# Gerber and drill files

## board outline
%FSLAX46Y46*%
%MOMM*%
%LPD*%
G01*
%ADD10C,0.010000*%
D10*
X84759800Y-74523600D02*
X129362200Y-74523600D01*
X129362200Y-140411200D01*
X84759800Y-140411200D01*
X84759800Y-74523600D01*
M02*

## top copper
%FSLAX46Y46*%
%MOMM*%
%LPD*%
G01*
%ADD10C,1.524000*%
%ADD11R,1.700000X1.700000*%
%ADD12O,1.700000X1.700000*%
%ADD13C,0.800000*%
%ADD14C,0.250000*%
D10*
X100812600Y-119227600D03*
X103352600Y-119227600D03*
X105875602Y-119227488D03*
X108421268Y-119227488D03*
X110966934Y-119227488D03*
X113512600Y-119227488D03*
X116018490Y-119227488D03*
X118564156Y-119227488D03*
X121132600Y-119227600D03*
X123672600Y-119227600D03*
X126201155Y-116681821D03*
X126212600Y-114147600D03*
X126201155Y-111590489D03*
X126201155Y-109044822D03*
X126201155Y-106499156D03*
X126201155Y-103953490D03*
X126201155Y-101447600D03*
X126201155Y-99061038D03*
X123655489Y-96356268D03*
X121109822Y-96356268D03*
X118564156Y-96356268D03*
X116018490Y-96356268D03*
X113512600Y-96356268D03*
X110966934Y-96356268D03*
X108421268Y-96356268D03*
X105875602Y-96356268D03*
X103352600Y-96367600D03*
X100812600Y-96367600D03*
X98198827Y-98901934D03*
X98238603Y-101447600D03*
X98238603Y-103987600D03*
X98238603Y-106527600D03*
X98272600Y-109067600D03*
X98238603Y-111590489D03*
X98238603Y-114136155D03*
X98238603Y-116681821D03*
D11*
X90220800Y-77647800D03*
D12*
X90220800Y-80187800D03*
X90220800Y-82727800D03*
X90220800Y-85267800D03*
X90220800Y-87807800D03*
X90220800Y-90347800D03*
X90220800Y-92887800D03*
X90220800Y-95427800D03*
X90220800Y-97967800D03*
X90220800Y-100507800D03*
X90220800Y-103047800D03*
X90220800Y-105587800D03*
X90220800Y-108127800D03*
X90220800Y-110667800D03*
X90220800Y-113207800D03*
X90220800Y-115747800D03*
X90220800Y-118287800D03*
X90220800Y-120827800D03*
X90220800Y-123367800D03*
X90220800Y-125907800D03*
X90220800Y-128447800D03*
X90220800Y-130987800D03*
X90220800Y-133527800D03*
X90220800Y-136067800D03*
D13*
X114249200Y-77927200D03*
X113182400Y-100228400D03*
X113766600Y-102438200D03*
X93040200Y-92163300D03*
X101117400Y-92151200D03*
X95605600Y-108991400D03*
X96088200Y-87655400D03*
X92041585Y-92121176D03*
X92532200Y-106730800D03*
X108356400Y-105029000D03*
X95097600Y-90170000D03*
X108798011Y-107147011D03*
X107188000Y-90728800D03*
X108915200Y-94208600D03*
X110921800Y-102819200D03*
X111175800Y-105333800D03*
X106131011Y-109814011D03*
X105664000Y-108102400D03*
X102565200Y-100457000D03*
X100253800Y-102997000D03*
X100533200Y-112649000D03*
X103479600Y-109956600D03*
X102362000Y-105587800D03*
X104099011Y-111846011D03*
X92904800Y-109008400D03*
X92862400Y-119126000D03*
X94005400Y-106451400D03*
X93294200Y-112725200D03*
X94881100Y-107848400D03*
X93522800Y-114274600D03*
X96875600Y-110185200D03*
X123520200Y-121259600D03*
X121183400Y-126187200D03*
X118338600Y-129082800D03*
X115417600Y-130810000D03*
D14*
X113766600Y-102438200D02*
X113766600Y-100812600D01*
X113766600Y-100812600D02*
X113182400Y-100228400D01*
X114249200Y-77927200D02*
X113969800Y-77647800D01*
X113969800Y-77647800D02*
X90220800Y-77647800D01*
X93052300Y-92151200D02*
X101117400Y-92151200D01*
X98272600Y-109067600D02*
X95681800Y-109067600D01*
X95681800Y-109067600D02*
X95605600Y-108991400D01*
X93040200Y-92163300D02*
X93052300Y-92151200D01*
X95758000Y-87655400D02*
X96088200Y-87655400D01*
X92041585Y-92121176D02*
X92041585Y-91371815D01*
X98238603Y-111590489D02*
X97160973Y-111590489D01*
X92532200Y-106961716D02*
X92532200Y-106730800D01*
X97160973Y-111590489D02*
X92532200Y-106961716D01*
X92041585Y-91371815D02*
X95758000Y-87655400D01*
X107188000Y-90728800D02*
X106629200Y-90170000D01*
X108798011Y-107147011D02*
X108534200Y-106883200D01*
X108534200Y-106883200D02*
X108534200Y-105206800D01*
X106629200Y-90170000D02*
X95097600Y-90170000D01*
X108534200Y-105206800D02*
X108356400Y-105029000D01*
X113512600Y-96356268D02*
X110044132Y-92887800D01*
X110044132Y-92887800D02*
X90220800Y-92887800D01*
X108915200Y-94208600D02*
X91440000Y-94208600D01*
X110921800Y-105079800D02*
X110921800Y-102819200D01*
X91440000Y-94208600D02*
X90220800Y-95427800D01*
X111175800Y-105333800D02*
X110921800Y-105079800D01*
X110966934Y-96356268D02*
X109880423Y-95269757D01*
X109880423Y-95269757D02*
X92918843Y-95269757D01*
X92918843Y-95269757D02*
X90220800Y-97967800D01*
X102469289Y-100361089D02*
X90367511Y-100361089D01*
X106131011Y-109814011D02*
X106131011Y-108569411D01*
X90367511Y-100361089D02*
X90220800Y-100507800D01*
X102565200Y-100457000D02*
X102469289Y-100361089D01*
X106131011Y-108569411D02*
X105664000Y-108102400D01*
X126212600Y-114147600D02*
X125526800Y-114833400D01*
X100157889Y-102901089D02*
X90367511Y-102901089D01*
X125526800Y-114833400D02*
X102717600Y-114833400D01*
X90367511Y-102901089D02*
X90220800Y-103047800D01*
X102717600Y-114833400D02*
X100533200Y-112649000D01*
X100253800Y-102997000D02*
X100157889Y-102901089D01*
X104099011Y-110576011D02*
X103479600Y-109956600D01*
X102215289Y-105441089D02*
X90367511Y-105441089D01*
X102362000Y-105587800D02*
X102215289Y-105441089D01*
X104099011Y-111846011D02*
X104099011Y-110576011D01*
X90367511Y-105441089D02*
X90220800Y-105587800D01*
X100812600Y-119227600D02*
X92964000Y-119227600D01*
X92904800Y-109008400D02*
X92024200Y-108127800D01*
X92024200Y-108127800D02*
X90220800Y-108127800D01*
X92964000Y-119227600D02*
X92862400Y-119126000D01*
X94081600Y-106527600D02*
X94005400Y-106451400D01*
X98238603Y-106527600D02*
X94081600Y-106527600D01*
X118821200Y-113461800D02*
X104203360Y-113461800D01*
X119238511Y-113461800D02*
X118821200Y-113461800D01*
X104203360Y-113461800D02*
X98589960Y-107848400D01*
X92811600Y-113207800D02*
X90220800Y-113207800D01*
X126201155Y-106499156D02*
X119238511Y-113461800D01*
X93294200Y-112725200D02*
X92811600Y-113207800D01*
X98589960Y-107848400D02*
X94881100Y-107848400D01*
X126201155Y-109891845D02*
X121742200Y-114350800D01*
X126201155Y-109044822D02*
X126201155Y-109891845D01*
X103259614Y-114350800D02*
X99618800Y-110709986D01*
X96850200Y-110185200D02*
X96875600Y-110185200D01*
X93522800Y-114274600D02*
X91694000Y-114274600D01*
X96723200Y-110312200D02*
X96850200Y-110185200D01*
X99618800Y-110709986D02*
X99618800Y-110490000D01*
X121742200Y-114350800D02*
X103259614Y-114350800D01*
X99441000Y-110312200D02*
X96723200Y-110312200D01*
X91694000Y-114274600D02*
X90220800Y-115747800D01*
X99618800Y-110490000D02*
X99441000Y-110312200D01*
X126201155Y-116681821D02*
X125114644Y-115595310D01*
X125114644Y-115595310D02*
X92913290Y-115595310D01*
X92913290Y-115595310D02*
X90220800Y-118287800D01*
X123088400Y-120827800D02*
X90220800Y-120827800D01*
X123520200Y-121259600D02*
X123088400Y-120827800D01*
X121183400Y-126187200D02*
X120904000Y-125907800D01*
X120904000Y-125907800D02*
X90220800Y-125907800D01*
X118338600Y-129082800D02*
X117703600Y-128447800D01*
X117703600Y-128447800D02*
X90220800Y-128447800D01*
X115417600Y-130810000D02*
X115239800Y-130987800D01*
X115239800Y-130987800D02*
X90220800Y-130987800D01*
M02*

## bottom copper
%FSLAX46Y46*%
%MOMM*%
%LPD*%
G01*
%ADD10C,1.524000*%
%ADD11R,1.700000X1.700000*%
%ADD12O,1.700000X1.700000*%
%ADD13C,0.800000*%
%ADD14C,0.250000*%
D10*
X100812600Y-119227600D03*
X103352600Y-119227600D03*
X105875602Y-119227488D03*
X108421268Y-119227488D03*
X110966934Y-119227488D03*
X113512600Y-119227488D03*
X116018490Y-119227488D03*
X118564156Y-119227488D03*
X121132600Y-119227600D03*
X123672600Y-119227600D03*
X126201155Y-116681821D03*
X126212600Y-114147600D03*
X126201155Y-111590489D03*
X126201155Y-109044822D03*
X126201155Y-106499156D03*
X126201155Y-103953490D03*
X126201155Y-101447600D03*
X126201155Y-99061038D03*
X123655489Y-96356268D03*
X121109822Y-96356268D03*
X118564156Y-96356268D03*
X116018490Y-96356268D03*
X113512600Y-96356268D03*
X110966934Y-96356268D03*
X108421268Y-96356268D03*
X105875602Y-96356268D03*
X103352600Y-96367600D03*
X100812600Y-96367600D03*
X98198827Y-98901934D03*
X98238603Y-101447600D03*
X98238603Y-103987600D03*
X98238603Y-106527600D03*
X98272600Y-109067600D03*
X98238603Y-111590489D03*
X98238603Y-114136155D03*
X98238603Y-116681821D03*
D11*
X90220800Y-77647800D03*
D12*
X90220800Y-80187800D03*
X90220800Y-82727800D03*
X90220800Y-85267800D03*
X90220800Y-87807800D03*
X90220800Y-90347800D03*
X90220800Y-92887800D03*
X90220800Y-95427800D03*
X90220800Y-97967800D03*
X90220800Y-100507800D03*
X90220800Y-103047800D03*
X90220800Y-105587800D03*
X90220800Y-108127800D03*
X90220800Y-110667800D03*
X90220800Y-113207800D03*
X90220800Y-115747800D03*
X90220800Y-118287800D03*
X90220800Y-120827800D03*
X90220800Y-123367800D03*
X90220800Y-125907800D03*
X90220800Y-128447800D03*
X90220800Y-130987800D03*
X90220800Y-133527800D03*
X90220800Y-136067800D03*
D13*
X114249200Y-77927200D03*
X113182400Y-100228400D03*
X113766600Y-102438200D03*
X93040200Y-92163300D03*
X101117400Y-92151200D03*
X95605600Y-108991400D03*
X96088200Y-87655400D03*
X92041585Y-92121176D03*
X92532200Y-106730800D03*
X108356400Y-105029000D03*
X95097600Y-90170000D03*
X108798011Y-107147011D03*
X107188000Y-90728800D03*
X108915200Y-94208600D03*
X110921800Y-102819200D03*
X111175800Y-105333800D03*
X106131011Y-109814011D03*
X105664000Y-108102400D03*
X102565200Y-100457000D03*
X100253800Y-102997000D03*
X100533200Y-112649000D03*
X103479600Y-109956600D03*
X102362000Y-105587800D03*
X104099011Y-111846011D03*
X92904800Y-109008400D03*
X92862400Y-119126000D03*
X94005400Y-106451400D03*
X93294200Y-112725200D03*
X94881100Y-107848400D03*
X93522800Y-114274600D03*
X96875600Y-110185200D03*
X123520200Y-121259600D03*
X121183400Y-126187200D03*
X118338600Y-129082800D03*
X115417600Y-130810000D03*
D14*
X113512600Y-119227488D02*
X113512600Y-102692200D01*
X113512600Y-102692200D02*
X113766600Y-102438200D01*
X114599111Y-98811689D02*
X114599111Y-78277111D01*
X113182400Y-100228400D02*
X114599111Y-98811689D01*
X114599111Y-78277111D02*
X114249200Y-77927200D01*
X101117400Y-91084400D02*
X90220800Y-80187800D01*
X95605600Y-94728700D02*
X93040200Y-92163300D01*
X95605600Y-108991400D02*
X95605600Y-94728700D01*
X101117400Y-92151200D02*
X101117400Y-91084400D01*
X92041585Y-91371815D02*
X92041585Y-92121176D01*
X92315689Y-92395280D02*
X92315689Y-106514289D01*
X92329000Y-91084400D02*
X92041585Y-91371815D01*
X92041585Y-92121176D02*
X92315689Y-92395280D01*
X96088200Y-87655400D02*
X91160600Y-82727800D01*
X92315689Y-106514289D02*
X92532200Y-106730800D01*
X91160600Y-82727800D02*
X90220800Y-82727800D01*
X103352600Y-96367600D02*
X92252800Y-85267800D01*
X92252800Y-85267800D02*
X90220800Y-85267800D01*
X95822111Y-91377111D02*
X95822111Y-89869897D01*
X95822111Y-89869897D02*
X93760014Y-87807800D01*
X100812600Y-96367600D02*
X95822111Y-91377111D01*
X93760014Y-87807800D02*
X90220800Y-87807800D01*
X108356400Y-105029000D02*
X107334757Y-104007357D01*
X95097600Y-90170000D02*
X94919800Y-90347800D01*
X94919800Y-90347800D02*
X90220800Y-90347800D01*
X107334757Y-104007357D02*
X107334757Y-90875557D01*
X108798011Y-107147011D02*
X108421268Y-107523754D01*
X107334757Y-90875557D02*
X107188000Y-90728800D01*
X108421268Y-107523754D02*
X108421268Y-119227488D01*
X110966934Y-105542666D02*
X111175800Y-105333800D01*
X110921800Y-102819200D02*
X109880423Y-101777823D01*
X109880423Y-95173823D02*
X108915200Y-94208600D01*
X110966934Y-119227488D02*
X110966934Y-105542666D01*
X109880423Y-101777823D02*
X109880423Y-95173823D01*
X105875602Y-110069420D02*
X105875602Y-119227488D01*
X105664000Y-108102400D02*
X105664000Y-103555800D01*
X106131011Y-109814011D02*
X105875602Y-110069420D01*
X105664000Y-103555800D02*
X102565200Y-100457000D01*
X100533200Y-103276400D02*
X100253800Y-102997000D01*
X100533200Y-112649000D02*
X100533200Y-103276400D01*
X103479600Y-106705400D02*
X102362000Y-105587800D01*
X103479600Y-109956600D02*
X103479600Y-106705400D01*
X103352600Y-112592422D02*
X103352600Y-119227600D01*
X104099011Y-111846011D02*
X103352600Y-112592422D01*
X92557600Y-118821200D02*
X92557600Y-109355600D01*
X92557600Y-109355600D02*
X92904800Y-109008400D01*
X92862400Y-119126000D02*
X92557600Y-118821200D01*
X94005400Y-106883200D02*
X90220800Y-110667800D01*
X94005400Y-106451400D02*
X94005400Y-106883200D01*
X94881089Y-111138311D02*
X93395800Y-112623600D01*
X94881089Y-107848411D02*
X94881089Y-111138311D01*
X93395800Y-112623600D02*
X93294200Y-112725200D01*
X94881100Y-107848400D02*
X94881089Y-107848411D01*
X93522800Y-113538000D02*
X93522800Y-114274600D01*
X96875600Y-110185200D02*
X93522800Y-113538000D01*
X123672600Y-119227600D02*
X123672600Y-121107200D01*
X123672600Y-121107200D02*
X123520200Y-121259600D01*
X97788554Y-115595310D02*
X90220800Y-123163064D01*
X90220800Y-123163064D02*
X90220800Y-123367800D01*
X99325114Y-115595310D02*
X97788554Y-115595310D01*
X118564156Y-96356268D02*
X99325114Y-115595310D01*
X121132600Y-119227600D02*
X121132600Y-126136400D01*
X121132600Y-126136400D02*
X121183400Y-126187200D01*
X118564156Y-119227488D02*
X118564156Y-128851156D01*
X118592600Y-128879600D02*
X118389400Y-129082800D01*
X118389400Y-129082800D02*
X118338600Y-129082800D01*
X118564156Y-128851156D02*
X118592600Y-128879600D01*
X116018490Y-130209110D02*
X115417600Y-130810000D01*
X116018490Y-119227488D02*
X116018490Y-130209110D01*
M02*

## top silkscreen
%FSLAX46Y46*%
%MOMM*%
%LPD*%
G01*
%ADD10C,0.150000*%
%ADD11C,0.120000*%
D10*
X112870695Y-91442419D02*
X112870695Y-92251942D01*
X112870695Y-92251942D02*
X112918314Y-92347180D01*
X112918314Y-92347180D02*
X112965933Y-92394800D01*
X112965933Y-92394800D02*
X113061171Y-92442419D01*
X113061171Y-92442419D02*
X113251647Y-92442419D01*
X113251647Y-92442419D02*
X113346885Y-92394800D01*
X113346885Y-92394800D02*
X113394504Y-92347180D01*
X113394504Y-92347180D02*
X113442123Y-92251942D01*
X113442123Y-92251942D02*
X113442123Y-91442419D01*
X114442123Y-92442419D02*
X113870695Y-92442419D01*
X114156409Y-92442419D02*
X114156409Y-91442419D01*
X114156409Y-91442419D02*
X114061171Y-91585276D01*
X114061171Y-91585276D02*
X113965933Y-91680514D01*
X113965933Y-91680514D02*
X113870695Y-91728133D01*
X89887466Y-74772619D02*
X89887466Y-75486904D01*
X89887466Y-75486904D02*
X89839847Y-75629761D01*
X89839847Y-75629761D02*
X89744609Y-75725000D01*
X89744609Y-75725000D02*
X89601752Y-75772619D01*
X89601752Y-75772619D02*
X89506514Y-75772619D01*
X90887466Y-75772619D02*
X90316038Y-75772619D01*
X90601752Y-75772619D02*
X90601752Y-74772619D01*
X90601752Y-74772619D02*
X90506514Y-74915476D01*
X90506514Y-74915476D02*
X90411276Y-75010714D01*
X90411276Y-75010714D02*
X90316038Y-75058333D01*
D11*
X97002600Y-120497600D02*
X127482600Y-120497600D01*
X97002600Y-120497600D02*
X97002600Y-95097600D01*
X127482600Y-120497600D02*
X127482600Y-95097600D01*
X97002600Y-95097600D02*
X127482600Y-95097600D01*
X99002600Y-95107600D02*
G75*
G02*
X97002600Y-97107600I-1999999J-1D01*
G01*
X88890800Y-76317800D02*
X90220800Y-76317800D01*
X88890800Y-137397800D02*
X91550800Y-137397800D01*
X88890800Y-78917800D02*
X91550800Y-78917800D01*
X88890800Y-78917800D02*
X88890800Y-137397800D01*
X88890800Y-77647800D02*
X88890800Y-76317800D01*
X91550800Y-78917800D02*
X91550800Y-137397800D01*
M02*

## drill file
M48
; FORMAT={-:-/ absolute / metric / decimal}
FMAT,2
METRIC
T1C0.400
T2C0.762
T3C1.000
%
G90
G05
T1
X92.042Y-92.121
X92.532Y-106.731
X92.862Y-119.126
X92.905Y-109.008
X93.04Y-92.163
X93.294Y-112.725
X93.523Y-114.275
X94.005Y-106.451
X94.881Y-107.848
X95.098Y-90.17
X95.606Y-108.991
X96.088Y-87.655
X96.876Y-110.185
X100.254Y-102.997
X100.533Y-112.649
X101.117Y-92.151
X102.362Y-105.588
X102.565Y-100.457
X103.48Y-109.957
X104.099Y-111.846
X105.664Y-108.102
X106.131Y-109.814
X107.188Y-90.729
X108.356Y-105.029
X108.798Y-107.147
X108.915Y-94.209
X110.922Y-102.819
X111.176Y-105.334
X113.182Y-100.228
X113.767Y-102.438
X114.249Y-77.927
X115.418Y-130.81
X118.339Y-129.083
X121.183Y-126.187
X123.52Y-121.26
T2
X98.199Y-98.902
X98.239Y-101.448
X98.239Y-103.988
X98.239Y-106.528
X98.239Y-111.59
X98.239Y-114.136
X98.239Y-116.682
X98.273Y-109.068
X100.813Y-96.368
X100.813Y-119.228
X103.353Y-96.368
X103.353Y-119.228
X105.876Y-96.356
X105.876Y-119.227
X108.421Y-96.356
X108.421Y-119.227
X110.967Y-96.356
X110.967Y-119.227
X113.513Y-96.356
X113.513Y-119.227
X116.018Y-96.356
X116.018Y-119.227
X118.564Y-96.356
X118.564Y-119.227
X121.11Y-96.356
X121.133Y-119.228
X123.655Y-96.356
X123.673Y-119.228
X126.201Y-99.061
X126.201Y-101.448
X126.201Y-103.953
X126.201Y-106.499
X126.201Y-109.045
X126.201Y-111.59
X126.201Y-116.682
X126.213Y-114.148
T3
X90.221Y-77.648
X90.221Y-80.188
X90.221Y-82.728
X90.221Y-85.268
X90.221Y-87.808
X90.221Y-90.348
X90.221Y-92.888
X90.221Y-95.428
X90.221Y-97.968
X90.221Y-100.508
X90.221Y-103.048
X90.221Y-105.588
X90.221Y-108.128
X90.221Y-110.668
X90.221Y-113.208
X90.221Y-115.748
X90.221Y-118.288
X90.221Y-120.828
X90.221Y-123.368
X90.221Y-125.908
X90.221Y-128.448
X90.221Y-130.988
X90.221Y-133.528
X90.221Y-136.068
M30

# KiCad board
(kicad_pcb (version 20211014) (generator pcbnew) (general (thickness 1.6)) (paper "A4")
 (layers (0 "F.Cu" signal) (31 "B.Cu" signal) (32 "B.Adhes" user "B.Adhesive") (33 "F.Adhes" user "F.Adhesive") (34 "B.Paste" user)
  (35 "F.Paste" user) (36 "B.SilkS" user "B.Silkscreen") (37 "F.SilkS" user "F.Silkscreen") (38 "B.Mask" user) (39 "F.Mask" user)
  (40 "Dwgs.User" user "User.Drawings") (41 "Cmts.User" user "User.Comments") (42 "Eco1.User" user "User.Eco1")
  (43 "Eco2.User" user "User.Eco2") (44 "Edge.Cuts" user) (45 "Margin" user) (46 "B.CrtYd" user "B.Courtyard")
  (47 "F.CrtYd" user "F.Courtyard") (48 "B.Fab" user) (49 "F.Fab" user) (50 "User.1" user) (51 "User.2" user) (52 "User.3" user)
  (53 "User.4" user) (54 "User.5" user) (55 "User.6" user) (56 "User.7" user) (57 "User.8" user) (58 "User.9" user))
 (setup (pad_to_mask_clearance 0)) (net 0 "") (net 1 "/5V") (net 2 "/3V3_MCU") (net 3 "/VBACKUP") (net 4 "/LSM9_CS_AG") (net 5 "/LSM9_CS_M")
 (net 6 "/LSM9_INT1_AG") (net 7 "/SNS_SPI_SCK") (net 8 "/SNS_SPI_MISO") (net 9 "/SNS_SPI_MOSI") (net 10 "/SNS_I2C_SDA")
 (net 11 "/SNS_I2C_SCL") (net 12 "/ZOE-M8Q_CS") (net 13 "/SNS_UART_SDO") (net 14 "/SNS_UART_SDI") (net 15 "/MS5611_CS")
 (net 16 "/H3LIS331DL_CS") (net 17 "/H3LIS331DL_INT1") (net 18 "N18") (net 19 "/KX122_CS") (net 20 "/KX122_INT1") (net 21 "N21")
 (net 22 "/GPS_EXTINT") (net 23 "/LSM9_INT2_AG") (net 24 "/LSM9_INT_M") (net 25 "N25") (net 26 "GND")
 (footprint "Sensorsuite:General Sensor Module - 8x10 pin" (layer "F.Cu") (at 113.5126 106.5276)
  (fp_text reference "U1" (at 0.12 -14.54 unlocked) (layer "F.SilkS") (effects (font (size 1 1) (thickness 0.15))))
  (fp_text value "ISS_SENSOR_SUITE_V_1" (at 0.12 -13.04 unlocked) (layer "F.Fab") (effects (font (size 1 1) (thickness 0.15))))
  (fp_line (start -16.51 13.97) (end 13.97 13.97) (layer "F.SilkS") (width 0.12))
  (fp_line (start -16.51 13.97) (end -16.51 -11.43) (layer "F.SilkS") (width 0.12))
  (fp_line (start 13.97 13.97) (end 13.97 -11.43) (layer "F.SilkS") (width 0.12))
  (fp_line (start -16.51 -11.43) (end 13.97 -11.43) (layer "F.SilkS") (width 0.12))
  (fp_arc (start -14.51 -11.42) (mid -15.095786 -10.005786) (end -16.51 -9.42) (layer "F.SilkS") (width 0.12))
  (pad "1" thru_hole circle (at -12.7 12.7) (size 1.524 1.524) (drill 0.762) (layers *.Cu *.Mask) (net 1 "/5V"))
  (pad "2" thru_hole circle (at -10.16 12.7) (size 1.524 1.524) (drill 0.762) (layers *.Cu *.Mask) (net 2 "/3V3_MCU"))
  (pad "3" thru_hole circle (at -7.636998 12.699888) (size 1.524 1.524) (drill 0.762) (layers *.Cu *.Mask) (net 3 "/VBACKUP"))
  (pad "4" thru_hole circle (at -5.091332 12.699888) (size 1.524 1.524) (drill 0.762) (layers *.Cu *.Mask) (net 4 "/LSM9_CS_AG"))
  (pad "5" thru_hole circle (at -2.545666 12.699888) (size 1.524 1.524) (drill 0.762) (layers *.Cu *.Mask) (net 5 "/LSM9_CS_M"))
  (pad "6" thru_hole circle (at 0 12.699888) (size 1.524 1.524) (drill 0.762) (layers *.Cu *.Mask) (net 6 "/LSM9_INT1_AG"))
  (pad "7" thru_hole circle (at 2.50589 12.699888) (size 1.524 1.524) (drill 0.762) (layers *.Cu *.Mask) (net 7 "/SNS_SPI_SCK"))
  (pad "8" thru_hole circle (at 5.051556 12.699888) (size 1.524 1.524) (drill 0.762) (layers *.Cu *.Mask) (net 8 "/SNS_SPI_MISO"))
  (pad "9" thru_hole circle (at 7.62 12.7) (size 1.524 1.524) (drill 0.762) (layers *.Cu *.Mask) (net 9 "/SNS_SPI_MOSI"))
  (pad "10" thru_hole circle (at 10.16 12.7) (size 1.524 1.524) (drill 0.762) (layers *.Cu *.Mask) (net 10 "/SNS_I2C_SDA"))
  (pad "11" thru_hole circle (at 12.688555 10.154221) (size 1.524 1.524) (drill 0.762) (layers *.Cu *.Mask) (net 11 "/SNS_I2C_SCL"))
  (pad "12" thru_hole circle (at 12.7 7.62) (size 1.524 1.524) (drill 0.762) (layers *.Cu *.Mask) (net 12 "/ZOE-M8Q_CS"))
  (pad "13" thru_hole circle (at 12.688555 5.062889) (size 1.524 1.524) (drill 0.762) (layers *.Cu *.Mask))
  (pad "14" thru_hole circle (at 12.688555 2.517222) (size 1.524 1.524) (drill 0.762) (layers *.Cu *.Mask) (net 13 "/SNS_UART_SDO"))
  (pad "15" thru_hole circle (at 12.688555 -0.028444) (size 1.524 1.524) (drill 0.762) (layers *.Cu *.Mask) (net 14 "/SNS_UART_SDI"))
  (pad "16" thru_hole circle (at 12.688555 -2.57411) (size 1.524 1.524) (drill 0.762) (layers *.Cu *.Mask))
  (pad "17" thru_hole circle (at 12.688555 -5.08) (size 1.524 1.524) (drill 0.762) (layers *.Cu *.Mask))
  (pad "18" thru_hole circle (at 12.688555 -7.466562) (size 1.524 1.524) (drill 0.762) (layers *.Cu *.Mask))
  (pad "19" thru_hole circle (at 10.142889 -10.171332) (size 1.524 1.524) (drill 0.762) (layers *.Cu *.Mask))
  (pad "20" thru_hole circle (at 7.597222 -10.171332) (size 1.524 1.524) (drill 0.762) (layers *.Cu *.Mask))
  (pad "21" thru_hole circle (at 5.051556 -10.171332) (size 1.524 1.524) (drill 0.762) (layers *.Cu *.Mask) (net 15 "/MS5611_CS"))
  (pad "22" thru_hole circle (at 2.50589 -10.171332) (size 1.524 1.524) (drill 0.762) (layers *.Cu *.Mask))
  (pad "23" thru_hole circle (at 0 -10.171332) (size 1.524 1.524) (drill 0.762) (layers *.Cu *.Mask) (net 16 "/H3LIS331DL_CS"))
  (pad "24" thru_hole circle (at -2.545666 -10.171332) (size 1.524 1.524) (drill 0.762) (layers *.Cu *.Mask) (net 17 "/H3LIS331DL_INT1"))
  (pad "25" thru_hole circle (at -5.091332 -10.171332) (size 1.524 1.524) (drill 0.762) (layers *.Cu *.Mask))
  (pad "26" thru_hole circle (at -7.636998 -10.171332) (size 1.524 1.524) (drill 0.762) (layers *.Cu *.Mask) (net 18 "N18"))
  (pad "27" thru_hole circle (at -10.16 -10.16) (size 1.524 1.524) (drill 0.762) (layers *.Cu *.Mask) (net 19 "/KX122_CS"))
  (pad "28" thru_hole circle (at -12.7 -10.16) (size 1.524 1.524) (drill 0.762) (layers *.Cu *.Mask) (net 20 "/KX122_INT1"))
  (pad "29" thru_hole circle (at -15.313773 -7.625666) (size 1.524 1.524) (drill 0.762) (layers *.Cu *.Mask))
  (pad "30" thru_hole circle (at -15.273997 -5.08) (size 1.524 1.524) (drill 0.762) (layers *.Cu *.Mask))
  (pad "31" thru_hole circle (at -15.273997 -2.54) (size 1.524 1.524) (drill 0.762) (layers *.Cu *.Mask) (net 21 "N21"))
  (pad "32" thru_hole circle (at -15.273997 0) (size 1.524 1.524) (drill 0.762) (layers *.Cu *.Mask) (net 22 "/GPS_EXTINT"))
  (pad "33" thru_hole circle (at -15.24 2.54) (size 1.524 1.524) (drill 0.762) (layers *.Cu *.Mask) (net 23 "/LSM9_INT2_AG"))
  (pad "34" thru_hole circle (at -15.273997 5.062889) (size 1.524 1.524) (drill 0.762) (layers *.Cu *.Mask) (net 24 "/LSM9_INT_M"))
  (pad "35" thru_hole circle (at -15.273997 7.608555) (size 1.524 1.524) (drill 0.762) (layers *.Cu *.Mask))
  (pad "36" thru_hole circle (at -15.273997 10.154221) (size 1.524 1.524) (drill 0.762) (layers *.Cu *.Mask)))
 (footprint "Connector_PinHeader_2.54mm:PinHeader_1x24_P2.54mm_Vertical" (layer "F.Cu") (at 90.2208 77.6478)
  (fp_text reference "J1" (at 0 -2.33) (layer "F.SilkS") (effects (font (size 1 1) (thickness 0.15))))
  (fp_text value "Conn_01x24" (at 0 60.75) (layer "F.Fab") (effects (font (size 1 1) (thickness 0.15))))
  (fp_line (start -1.33 -1.33) (end 0 -1.33) (layer "F.SilkS") (width 0.12))
  (fp_line (start -1.33 59.75) (end 1.33 59.75) (layer "F.SilkS") (width 0.12))
  (fp_line (start -1.33 1.27) (end 1.33 1.27) (layer "F.SilkS") (width 0.12))
  (fp_line (start -1.33 1.27) (end -1.33 59.75) (layer "F.SilkS") (width 0.12))
  (fp_line (start -1.33 0) (end -1.33 -1.33) (layer "F.SilkS") (width 0.12))
  (fp_line (start 1.33 1.27) (end 1.33 59.75) (layer "F.SilkS") (width 0.12))
  (pad "1" thru_hole rect locked (at 0 0) (size 1.7 1.7) (drill 1) (layers *.Cu *.Mask) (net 6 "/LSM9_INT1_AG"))
  (pad "2" thru_hole oval locked (at 0 2.54) (size 1.7 1.7) (drill 1) (layers *.Cu *.Mask) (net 23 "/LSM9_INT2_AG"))
  (pad "3" thru_hole oval locked (at 0 5.08) (size 1.7 1.7) (drill 1) (layers *.Cu *.Mask) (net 24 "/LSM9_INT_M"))
  (pad "4" thru_hole oval locked (at 0 7.62) (size 1.7 1.7) (drill 1) (layers *.Cu *.Mask) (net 19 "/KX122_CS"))
  (pad "5" thru_hole oval locked (at 0 10.16) (size 1.7 1.7) (drill 1) (layers *.Cu *.Mask) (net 20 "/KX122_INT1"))
  (pad "6" thru_hole oval locked (at 0 12.7) (size 1.7 1.7) (drill 1) (layers *.Cu *.Mask) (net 4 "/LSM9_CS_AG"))
  (pad "7" thru_hole oval locked (at 0 15.24) (size 1.7 1.7) (drill 1) (layers *.Cu *.Mask) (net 16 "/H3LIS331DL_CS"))
  (pad "8" thru_hole oval locked (at 0 17.78) (size 1.7 1.7) (drill 1) (layers *.Cu *.Mask) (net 5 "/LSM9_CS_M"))
  (pad "9" thru_hole oval locked (at 0 20.32) (size 1.7 1.7) (drill 1) (layers *.Cu *.Mask) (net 17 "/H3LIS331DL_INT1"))
  (pad "10" thru_hole oval locked (at 0 22.86) (size 1.7 1.7) (drill 1) (layers *.Cu *.Mask) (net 3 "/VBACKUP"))
  (pad "11" thru_hole oval locked (at 0 25.4) (size 1.7 1.7) (drill 1) (layers *.Cu *.Mask) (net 12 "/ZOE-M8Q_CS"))
  (pad "12" thru_hole oval locked (at 0 27.94) (size 1.7 1.7) (drill 1) (layers *.Cu *.Mask) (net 2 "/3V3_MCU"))
  (pad "13" thru_hole oval locked (at 0 30.48) (size 1.7 1.7) (drill 1) (layers *.Cu *.Mask) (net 1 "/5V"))
  (pad "14" thru_hole oval locked (at 0 33.02) (size 1.7 1.7) (drill 1) (layers *.Cu *.Mask) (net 22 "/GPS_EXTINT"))
  (pad "15" thru_hole oval locked (at 0 35.56) (size 1.7 1.7) (drill 1) (layers *.Cu *.Mask) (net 14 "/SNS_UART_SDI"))
  (pad "16" thru_hole oval locked (at 0 38.1) (size 1.7 1.7) (drill 1) (layers *.Cu *.Mask) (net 13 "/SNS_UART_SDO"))
  (pad "17" thru_hole oval locked (at 0 40.64) (size 1.7 1.7) (drill 1) (layers *.Cu *.Mask) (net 11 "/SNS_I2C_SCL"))
  (pad "18" thru_hole oval locked (at 0 43.18) (size 1.7 1.7) (drill 1) (layers *.Cu *.Mask) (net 10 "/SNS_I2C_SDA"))
  (pad "19" thru_hole oval locked (at 0 45.72) (size 1.7 1.7) (drill 1) (layers *.Cu *.Mask) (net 15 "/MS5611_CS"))
  (pad "20" thru_hole oval locked (at 0 48.26) (size 1.7 1.7) (drill 1) (layers *.Cu *.Mask) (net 9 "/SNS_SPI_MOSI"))
  (pad "21" thru_hole oval locked (at 0 50.8) (size 1.7 1.7) (drill 1) (layers *.Cu *.Mask) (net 8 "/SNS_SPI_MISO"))
  (pad "22" thru_hole oval locked (at 0 53.34) (size 1.7 1.7) (drill 1) (layers *.Cu *.Mask) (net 7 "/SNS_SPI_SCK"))
  (pad "23" thru_hole oval locked (at 0 55.88) (size 1.7 1.7) (drill 1) (layers *.Cu *.Mask) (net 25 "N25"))
  (pad "24" thru_hole oval locked (at 0 58.42) (size 1.7 1.7) (drill 1) (layers *.Cu *.Mask) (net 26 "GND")))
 (gr_rect (start 84.7598 74.5236) (end 129.3622 140.4112) (layer "Edge.Cuts") (width 0.01) (fill none))
 (segment (start 113.7666 102.4382) (end 113.7666 100.8126) (width 0.25) (layer "F.Cu") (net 6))
 (segment (start 113.7666 100.8126) (end 113.1824 100.2284) (width 0.25) (layer "F.Cu") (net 6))
 (segment (start 114.2492 77.9272) (end 113.9698 77.6478) (width 0.25) (layer "F.Cu") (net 6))
 (segment (start 113.9698 77.6478) (end 90.2208 77.6478) (width 0.25) (layer "F.Cu") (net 6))
 (via (at 114.2492 77.9272) (size 0.8) (drill 0.4) (layers "F.Cu" "B.Cu") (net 6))
 (via (at 113.1824 100.2284) (size 0.8) (drill 0.4) (layers "F.Cu" "B.Cu") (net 6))
 (via (at 113.7666 102.4382) (size 0.8) (drill 0.4) (layers "F.Cu" "B.Cu") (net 6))
 (segment (start 113.5126 119.227488) (end 113.5126 102.6922) (width 0.25) (layer "B.Cu") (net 6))
 (segment (start 113.5126 102.6922) (end 113.7666 102.4382) (width 0.25) (layer "B.Cu") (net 6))
 (segment (start 114.599111 98.811689) (end 114.599111 78.277111) (width 0.25) (layer "B.Cu") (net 6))
 (segment (start 113.1824 100.2284) (end 114.599111 98.811689) (width 0.25) (layer "B.Cu") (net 6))
 (segment (start 114.599111 78.277111) (end 114.2492 77.9272) (width 0.25) (layer "B.Cu") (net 6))
 (segment (start 93.0523 92.1512) (end 101.1174 92.1512) (width 0.25) (layer "F.Cu") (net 23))
 (segment (start 98.2726 109.0676) (end 95.6818 109.0676) (width 0.25) (layer "F.Cu") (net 23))
 (segment (start 95.6818 109.0676) (end 95.6056 108.9914) (width 0.25) (layer "F.Cu") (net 23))
 (segment (start 93.0402 92.1633) (end 93.0523 92.1512) (width 0.25) (layer "F.Cu") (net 23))
 (via (at 93.0402 92.1633) (size 0.8) (drill 0.4) (layers "F.Cu" "B.Cu") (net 23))
 (via (at 101.1174 92.1512) (size 0.8) (drill 0.4) (layers "F.Cu" "B.Cu") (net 23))
 (via (at 95.6056 108.9914) (size 0.8) (drill 0.4) (layers "F.Cu" "B.Cu") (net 23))
 (segment (start 101.1174 91.0844) (end 90.2208 80.1878) (width 0.25) (layer "B.Cu") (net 23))
 (segment (start 95.6056 94.7287) (end 93.0402 92.1633) (width 0.25) (layer "B.Cu") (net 23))
 (segment (start 95.6056 108.9914) (end 95.6056 94.7287) (width 0.25) (layer "B.Cu") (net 23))
 (segment (start 101.1174 92.1512) (end 101.1174 91.0844) (width 0.25) (layer "B.Cu") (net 23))
 (segment (start 95.758 87.6554) (end 96.0882 87.6554) (width 0.25) (layer "F.Cu") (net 24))
 (segment (start 92.041585 92.121176) (end 92.041585 91.371815) (width 0.25) (layer "F.Cu") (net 24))
 (segment (start 98.238603 111.590489) (end 97.160973 111.590489) (width 0.25) (layer "F.Cu") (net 24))
 (segment (start 92.5322 106.961716) (end 92.5322 106.7308) (width 0.25) (layer "F.Cu") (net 24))
 (segment (start 97.160973 111.590489) (end 92.5322 106.961716) (width 0.25) (layer "F.Cu") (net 24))
 (segment (start 92.041585 91.371815) (end 95.758 87.6554) (width 0.25) (layer "F.Cu") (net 24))
 (via (at 96.0882 87.6554) (size 0.8) (drill 0.4) (layers "F.Cu" "B.Cu") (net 24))
 (via (at 92.041585 92.121176) (size 0.8) (drill 0.4) (layers "F.Cu" "B.Cu") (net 24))
 (via (at 92.5322 106.7308) (size 0.8) (drill 0.4) (layers "F.Cu" "B.Cu") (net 24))
 (segment (start 92.041585 91.371815) (end 92.041585 92.121176) (width 0.25) (layer "B.Cu") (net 24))
 (segment (start 92.315689 92.39528) (end 92.315689 106.514289) (width 0.25) (layer "B.Cu") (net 24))
 (segment (start 92.329 91.0844) (end 92.041585 91.371815) (width 0.25) (layer "B.Cu") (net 24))
 (segment (start 92.041585 92.121176) (end 92.315689 92.39528) (width 0.25) (layer "B.Cu") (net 24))
 (segment (start 96.0882 87.6554) (end 91.1606 82.7278) (width 0.25) (layer "B.Cu") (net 24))
 (segment (start 92.315689 106.514289) (end 92.5322 106.7308) (width 0.25) (layer "B.Cu") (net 24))
 (segment (start 91.1606 82.7278) (end 90.2208 82.7278) (width 0.25) (layer "B.Cu") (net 24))
 (segment (start 103.3526 96.3676) (end 92.2528 85.2678) (width 0.25) (layer "B.Cu") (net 19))
 (segment (start 92.2528 85.2678) (end 90.2208 85.2678) (width 0.25) (layer "B.Cu") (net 19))
 (segment (start 95.822111 91.377111) (end 95.822111 89.869897) (width 0.25) (layer "B.Cu") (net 20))
 (segment (start 95.822111 89.869897) (end 93.760014 87.8078) (width 0.25) (layer "B.Cu") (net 20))
 (segment (start 100.8126 96.3676) (end 95.822111 91.377111) (width 0.25) (layer "B.Cu") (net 20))
 (segment (start 93.760014 87.8078) (end 90.2208 87.8078) (width 0.25) (layer "B.Cu") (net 20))
 (segment (start 107.188 90.7288) (end 106.6292 90.17) (width 0.25) (layer "F.Cu") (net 4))
 (segment (start 108.798011 107.147011) (end 108.5342 106.8832) (width 0.25) (layer "F.Cu") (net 4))
 (segment (start 108.5342 106.8832) (end 108.5342 105.2068) (width 0.25) (layer "F.Cu") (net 4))
 (segment (start 106.6292 90.17) (end 95.0976 90.17) (width 0.25) (layer "F.Cu") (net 4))
 (segment (start 108.5342 105.2068) (end 108.3564 105.029) (width 0.25) (layer "F.Cu") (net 4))
 (via (at 108.3564 105.029) (size 0.8) (drill 0.4) (layers "F.Cu" "B.Cu") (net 4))
 (via (at 95.0976 90.17) (size 0.8) (drill 0.4) (layers "F.Cu" "B.Cu") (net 4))
 (via (at 108.798011 107.147011) (size 0.8) (drill 0.4) (layers "F.Cu" "B.Cu") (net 4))
 (via (at 107.188 90.7288) (size 0.8) (drill 0.4) (layers "F.Cu" "B.Cu") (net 4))
 (segment (start 108.3564 105.029) (end 107.334757 104.007357) (width 0.25) (layer "B.Cu") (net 4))
 (segment (start 95.0976 90.17) (end 94.9198 90.3478) (width 0.25) (layer "B.Cu") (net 4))
 (segment (start 94.9198 90.3478) (end 90.2208 90.3478) (width 0.25) (layer "B.Cu") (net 4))
 (segment (start 107.334757 104.007357) (end 107.334757 90.875557) (width 0.25) (layer "B.Cu") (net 4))
 (segment (start 108.798011 107.147011) (end 108.421268 107.523754) (width 0.25) (layer "B.Cu") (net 4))
 (segment (start 107.334757 90.875557) (end 107.188 90.7288) (width 0.25) (layer "B.Cu") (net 4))
 (segment (start 108.421268 107.523754) (end 108.421268 119.227488) (width 0.25) (layer "B.Cu") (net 4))
 (segment (start 113.5126 96.356268) (end 110.044132 92.8878) (width 0.25) (layer "F.Cu") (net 16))
 (segment (start 110.044132 92.8878) (end 90.2208 92.8878) (width 0.25) (layer "F.Cu") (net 16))
 (segment (start 108.9152 94.2086) (end 91.44 94.2086) (width 0.25) (layer "F.Cu") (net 5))
 (segment (start 110.9218 105.0798) (end 110.9218 102.8192) (width 0.25) (layer "F.Cu") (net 5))
 (segment (start 91.44 94.2086) (end 90.2208 95.4278) (width 0.25) (layer "F.Cu") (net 5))
 (segment (start 111.1758 105.3338) (end 110.9218 105.0798) (width 0.25) (layer "F.Cu") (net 5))
 (via (at 108.9152 94.2086) (size 0.8) (drill 0.4) (layers "F.Cu" "B.Cu") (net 5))
 (via (at 110.9218 102.8192) (size 0.8) (drill 0.4) (layers "F.Cu" "B.Cu") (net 5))
 (via (at 111.1758 105.3338) (size 0.8) (drill 0.4) (layers "F.Cu" "B.Cu") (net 5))
 (segment (start 110.966934 105.542666) (end 111.1758 105.3338) (width 0.25) (layer "B.Cu") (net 5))
 (segment (start 110.9218 102.8192) (end 109.880423 101.777823) (width 0.25) (layer "B.Cu") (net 5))
 (segment (start 109.880423 95.173823) (end 108.9152 94.2086) (width 0.25) (layer "B.Cu") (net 5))
 (segment (start 110.966934 119.227488) (end 110.966934 105.542666) (width 0.25) (layer "B.Cu") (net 5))
 (segment (start 109.880423 101.777823) (end 109.880423 95.173823) (width 0.25) (layer "B.Cu") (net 5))
 (segment (start 110.966934 96.356268) (end 109.880423 95.269757) (width 0.25) (layer "F.Cu") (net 17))
 (segment (start 109.880423 95.269757) (end 92.918843 95.269757) (width 0.25) (layer "F.Cu") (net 17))
 (segment (start 92.918843 95.269757) (end 90.2208 97.9678) (width 0.25) (layer "F.Cu") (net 17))
 (segment (start 102.469289 100.361089) (end 90.367511 100.361089) (width 0.25) (layer "F.Cu") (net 3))
 (segment (start 106.131011 109.814011) (end 106.131011 108.569411) (width 0.25) (layer "F.Cu") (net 3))
 (segment (start 90.367511 100.361089) (end 90.2208 100.5078) (width 0.25) (layer "F.Cu") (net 3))
 (segment (start 102.5652 100.457) (end 102.469289 100.361089) (width 0.25) (layer "F.Cu") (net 3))
 (segment (start 106.131011 108.569411) (end 105.664 108.1024) (width 0.25) (layer "F.Cu") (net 3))
 (via (at 106.131011 109.814011) (size 0.8) (drill 0.4) (layers "F.Cu" "B.Cu") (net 3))
 (via (at 105.664 108.1024) (size 0.8) (drill 0.4) (layers "F.Cu" "B.Cu") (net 3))
 (via (at 102.5652 100.457) (size 0.8) (drill 0.4) (layers "F.Cu" "B.Cu") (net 3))
 (segment (start 105.875602 110.06942) (end 105.875602 119.227488) (width 0.25) (layer "B.Cu") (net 3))
 (segment (start 105.664 108.1024) (end 105.664 103.5558) (width 0.25) (layer "B.Cu") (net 3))
 (segment (start 106.131011 109.814011) (end 105.875602 110.06942) (width 0.25) (layer "B.Cu") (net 3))
 (segment (start 105.664 103.5558) (end 102.5652 100.457) (width 0.25) (layer "B.Cu") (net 3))
 (segment (start 126.2126 114.1476) (end 125.5268 114.8334) (width 0.25) (layer "F.Cu") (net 12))
 (segment (start 100.157889 102.901089) (end 90.367511 102.901089) (width 0.25) (layer "F.Cu") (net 12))
 (segment (start 125.5268 114.8334) (end 102.7176 114.8334) (width 0.25) (layer "F.Cu") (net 12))
 (segment (start 90.367511 102.901089) (end 90.2208 103.0478) (width 0.25) (layer "F.Cu") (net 12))
 (segment (start 102.7176 114.8334) (end 100.5332 112.649) (width 0.25) (layer "F.Cu") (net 12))
 (segment (start 100.2538 102.997) (end 100.157889 102.901089) (width 0.25) (layer "F.Cu") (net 12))
 (via (at 100.2538 102.997) (size 0.8) (drill 0.4) (layers "F.Cu" "B.Cu") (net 12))
 (via (at 100.5332 112.649) (size 0.8) (drill 0.4) (layers "F.Cu" "B.Cu") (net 12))
 (segment (start 100.5332 103.2764) (end 100.2538 102.997) (width 0.25) (layer "B.Cu") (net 12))
 (segment (start 100.5332 112.649) (end 100.5332 103.2764) (width 0.25) (layer "B.Cu") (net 12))
 (segment (start 104.099011 110.576011) (end 103.4796 109.9566) (width 0.25) (layer "F.Cu") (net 2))
 (segment (start 102.215289 105.441089) (end 90.367511 105.441089) (width 0.25) (layer "F.Cu") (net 2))
 (segment (start 102.362 105.5878) (end 102.215289 105.441089) (width 0.25) (layer "F.Cu") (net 2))
 (segment (start 104.099011 111.846011) (end 104.099011 110.576011) (width 0.25) (layer "F.Cu") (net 2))
 (segment (start 90.367511 105.441089) (end 90.2208 105.5878) (width 0.25) (layer "F.Cu") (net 2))
 (via (at 103.4796 109.9566) (size 0.8) (drill 0.4) (layers "F.Cu" "B.Cu") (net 2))
 (via (at 102.362 105.5878) (size 0.8) (drill 0.4) (layers "F.Cu" "B.Cu") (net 2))
 (via (at 104.099011 111.846011) (size 0.8) (drill 0.4) (layers "F.Cu" "B.Cu") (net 2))
 (segment (start 103.4796 106.7054) (end 102.362 105.5878) (width 0.25) (layer "B.Cu") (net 2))
 (segment (start 103.4796 109.9566) (end 103.4796 106.7054) (width 0.25) (layer "B.Cu") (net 2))
 (segment (start 103.3526 112.592422) (end 103.3526 119.2276) (width 0.25) (layer "B.Cu") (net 2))
 (segment (start 104.099011 111.846011) (end 103.3526 112.592422) (width 0.25) (layer "B.Cu") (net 2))
 (segment (start 100.8126 119.2276) (end 92.964 119.2276) (width 0.25) (layer "F.Cu") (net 1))
 (segment (start 92.9048 109.0084) (end 92.0242 108.1278) (width 0.25) (layer "F.Cu") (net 1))
 (segment (start 92.0242 108.1278) (end 90.2208 108.1278) (width 0.25) (layer "F.Cu") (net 1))
 (segment (start 92.964 119.2276) (end 92.8624 119.126) (width 0.25) (layer "F.Cu") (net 1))
 (via (at 92.9048 109.0084) (size 0.8) (drill 0.4) (layers "F.Cu" "B.Cu") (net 1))
 (via (at 92.8624 119.126) (size 0.8) (drill 0.4) (layers "F.Cu" "B.Cu") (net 1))
 (segment (start 92.5576 118.8212) (end 92.5576 109.3556) (width 0.25) (layer "B.Cu") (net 1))
 (segment (start 92.5576 109.3556) (end 92.9048 109.0084) (width 0.25) (layer "B.Cu") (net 1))
 (segment (start 92.8624 119.126) (end 92.5576 118.8212) (width 0.25) (layer "B.Cu") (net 1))
 (segment (start 94.0816 106.5276) (end 94.0054 106.4514) (width 0.25) (layer "F.Cu") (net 22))
 (segment (start 98.238603 106.5276) (end 94.0816 106.5276) (width 0.25) (layer "F.Cu") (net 22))
 (via (at 94.0054 106.4514) (size 0.8) (drill 0.4) (layers "F.Cu" "B.Cu") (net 22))
 (segment (start 94.0054 106.8832) (end 90.2208 110.6678) (width 0.25) (layer "B.Cu") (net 22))
 (segment (start 94.0054 106.4514) (end 94.0054 106.8832) (width 0.25) (layer "B.Cu") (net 22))
 (segment (start 118.8212 113.4618) (end 104.20336 113.4618) (width 0.25) (layer "F.Cu") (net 14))
 (segment (start 119.238511 113.4618) (end 118.8212 113.4618) (width 0.25) (layer "F.Cu") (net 14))
 (segment (start 104.20336 113.4618) (end 98.58996 107.8484) (width 0.25) (layer "F.Cu") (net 14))
 (segment (start 92.8116 113.2078) (end 90.2208 113.2078) (width 0.25) (layer "F.Cu") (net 14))
 (segment (start 126.201155 106.499156) (end 119.238511 113.4618) (width 0.25) (layer "F.Cu") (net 14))
 (segment (start 93.2942 112.7252) (end 92.8116 113.2078) (width 0.25) (layer "F.Cu") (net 14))
 (segment (start 98.58996 107.8484) (end 94.8811 107.8484) (width 0.25) (layer "F.Cu") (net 14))
 (via (at 93.2942 112.7252) (size 0.8) (drill 0.4) (layers "F.Cu" "B.Cu") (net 14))
 (via (at 94.8811 107.8484) (size 0.8) (drill 0.4) (layers "F.Cu" "B.Cu") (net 14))
 (segment (start 94.881089 111.138311) (end 93.3958 112.6236) (width 0.25) (layer "B.Cu") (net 14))
 (segment (start 94.881089 107.848411) (end 94.881089 111.138311) (width 0.25) (layer "B.Cu") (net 14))
 (segment (start 93.3958 112.6236) (end 93.2942 112.7252) (width 0.25) (layer "B.Cu") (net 14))
 (segment (start 94.8811 107.8484) (end 94.881089 107.848411) (width 0.25) (layer "B.Cu") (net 14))
 (segment (start 126.201155 109.891845) (end 121.7422 114.3508) (width 0.25) (layer "F.Cu") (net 13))
 (segment (start 126.201155 109.044822) (end 126.201155 109.891845) (width 0.25) (layer "F.Cu") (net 13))
 (segment (start 103.259614 114.3508) (end 99.6188 110.709986) (width 0.25) (layer "F.Cu") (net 13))
 (segment (start 96.8502 110.1852) (end 96.8756 110.1852) (width 0.25) (layer "F.Cu") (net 13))
 (segment (start 93.5228 114.2746) (end 91.694 114.2746) (width 0.25) (layer "F.Cu") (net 13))
 (segment (start 96.7232 110.3122) (end 96.8502 110.1852) (width 0.25) (layer "F.Cu") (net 13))
 (segment (start 99.6188 110.709986) (end 99.6188 110.49) (width 0.25) (layer "F.Cu") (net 13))
 (segment (start 121.7422 114.3508) (end 103.259614 114.3508) (width 0.25) (layer "F.Cu") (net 13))
 (segment (start 99.441 110.3122) (end 96.7232 110.3122) (width 0.25) (layer "F.Cu") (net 13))
 (segment (start 91.694 114.2746) (end 90.2208 115.7478) (width 0.25) (layer "F.Cu") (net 13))
 (segment (start 99.6188 110.49) (end 99.441 110.3122) (width 0.25) (layer "F.Cu") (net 13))
 (via (at 93.5228 114.2746) (size 0.8) (drill 0.4) (layers "F.Cu" "B.Cu") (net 13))
 (via (at 96.8756 110.1852) (size 0.8) (drill 0.4) (layers "F.Cu" "B.Cu") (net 13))
 (segment (start 93.5228 113.538) (end 93.5228 114.2746) (width 0.25) (layer "B.Cu") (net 13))
 (segment (start 96.8756 110.1852) (end 93.5228 113.538) (width 0.25) (layer "B.Cu") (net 13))
 (segment (start 126.201155 116.681821) (end 125.114644 115.59531) (width 0.25) (layer "F.Cu") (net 11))
 (segment (start 125.114644 115.59531) (end 92.91329 115.59531) (width 0.25) (layer "F.Cu") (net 11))
 (segment (start 92.91329 115.59531) (end 90.2208 118.2878) (width 0.25) (layer "F.Cu") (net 11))
 (segment (start 123.0884 120.8278) (end 90.2208 120.8278) (width 0.25) (layer "F.Cu") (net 10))
 (segment (start 123.5202 121.2596) (end 123.0884 120.8278) (width 0.25) (layer "F.Cu") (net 10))
 (via (at 123.5202 121.2596) (size 0.8) (drill 0.4) (layers "F.Cu" "B.Cu") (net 10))
 (segment (start 123.6726 119.2276) (end 123.6726 121.1072) (width 0.25) (layer "B.Cu") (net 10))
 (segment (start 123.6726 121.1072) (end 123.5202 121.2596) (width 0.25) (layer "B.Cu") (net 10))
 (segment (start 97.788554 115.59531) (end 90.2208 123.163064) (width 0.25) (layer "B.Cu") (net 15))
 (segment (start 90.2208 123.163064) (end 90.2208 123.3678) (width 0.25) (layer "B.Cu") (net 15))
 (segment (start 99.325114 115.59531) (end 97.788554 115.59531) (width 0.25) (layer "B.Cu") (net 15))
 (segment (start 118.564156 96.356268) (end 99.325114 115.59531) (width 0.25) (layer "B.Cu") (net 15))
 (segment (start 121.1834 126.1872) (end 120.904 125.9078) (width 0.25) (layer "F.Cu") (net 9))
 (segment (start 120.904 125.9078) (end 90.2208 125.9078) (width 0.25) (layer "F.Cu") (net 9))
 (via (at 121.1834 126.1872) (size 0.8) (drill 0.4) (layers "F.Cu" "B.Cu") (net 9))
 (segment (start 121.1326 119.2276) (end 121.1326 126.1364) (width 0.25) (layer "B.Cu") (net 9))
 (segment (start 121.1326 126.1364) (end 121.1834 126.1872) (width 0.25) (layer "B.Cu") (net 9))
 (segment (start 118.3386 129.0828) (end 117.7036 128.4478) (width 0.25) (layer "F.Cu") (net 8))
 (segment (start 117.7036 128.4478) (end 90.2208 128.4478) (width 0.25) (layer "F.Cu") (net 8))
 (via (at 118.3386 129.0828) (size 0.8) (drill 0.4) (layers "F.Cu" "B.Cu") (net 8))
 (segment (start 118.564156 119.227488) (end 118.564156 128.851156) (width 0.25) (layer "B.Cu") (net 8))
 (segment (start 118.5926 128.8796) (end 118.3894 129.0828) (width 0.25) (layer "B.Cu") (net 8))
 (segment (start 118.3894 129.0828) (end 118.3386 129.0828) (width 0.25) (layer "B.Cu") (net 8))
 (segment (start 118.564156 128.851156) (end 118.5926 128.8796) (width 0.25) (layer "B.Cu") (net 8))
 (segment (start 115.4176 130.81) (end 115.2398 130.9878) (width 0.25) (layer "F.Cu") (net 7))
 (segment (start 115.2398 130.9878) (end 90.2208 130.9878) (width 0.25) (layer "F.Cu") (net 7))
 (via (at 115.4176 130.81) (size 0.8) (drill 0.4) (layers "F.Cu" "B.Cu") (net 7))
 (segment (start 116.01849 130.20911) (end 115.4176 130.81) (width 0.25) (layer "B.Cu") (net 7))
 (segment (start 116.01849 119.227488) (end 116.01849 130.20911) (width 0.25) (layer "B.Cu") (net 7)))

